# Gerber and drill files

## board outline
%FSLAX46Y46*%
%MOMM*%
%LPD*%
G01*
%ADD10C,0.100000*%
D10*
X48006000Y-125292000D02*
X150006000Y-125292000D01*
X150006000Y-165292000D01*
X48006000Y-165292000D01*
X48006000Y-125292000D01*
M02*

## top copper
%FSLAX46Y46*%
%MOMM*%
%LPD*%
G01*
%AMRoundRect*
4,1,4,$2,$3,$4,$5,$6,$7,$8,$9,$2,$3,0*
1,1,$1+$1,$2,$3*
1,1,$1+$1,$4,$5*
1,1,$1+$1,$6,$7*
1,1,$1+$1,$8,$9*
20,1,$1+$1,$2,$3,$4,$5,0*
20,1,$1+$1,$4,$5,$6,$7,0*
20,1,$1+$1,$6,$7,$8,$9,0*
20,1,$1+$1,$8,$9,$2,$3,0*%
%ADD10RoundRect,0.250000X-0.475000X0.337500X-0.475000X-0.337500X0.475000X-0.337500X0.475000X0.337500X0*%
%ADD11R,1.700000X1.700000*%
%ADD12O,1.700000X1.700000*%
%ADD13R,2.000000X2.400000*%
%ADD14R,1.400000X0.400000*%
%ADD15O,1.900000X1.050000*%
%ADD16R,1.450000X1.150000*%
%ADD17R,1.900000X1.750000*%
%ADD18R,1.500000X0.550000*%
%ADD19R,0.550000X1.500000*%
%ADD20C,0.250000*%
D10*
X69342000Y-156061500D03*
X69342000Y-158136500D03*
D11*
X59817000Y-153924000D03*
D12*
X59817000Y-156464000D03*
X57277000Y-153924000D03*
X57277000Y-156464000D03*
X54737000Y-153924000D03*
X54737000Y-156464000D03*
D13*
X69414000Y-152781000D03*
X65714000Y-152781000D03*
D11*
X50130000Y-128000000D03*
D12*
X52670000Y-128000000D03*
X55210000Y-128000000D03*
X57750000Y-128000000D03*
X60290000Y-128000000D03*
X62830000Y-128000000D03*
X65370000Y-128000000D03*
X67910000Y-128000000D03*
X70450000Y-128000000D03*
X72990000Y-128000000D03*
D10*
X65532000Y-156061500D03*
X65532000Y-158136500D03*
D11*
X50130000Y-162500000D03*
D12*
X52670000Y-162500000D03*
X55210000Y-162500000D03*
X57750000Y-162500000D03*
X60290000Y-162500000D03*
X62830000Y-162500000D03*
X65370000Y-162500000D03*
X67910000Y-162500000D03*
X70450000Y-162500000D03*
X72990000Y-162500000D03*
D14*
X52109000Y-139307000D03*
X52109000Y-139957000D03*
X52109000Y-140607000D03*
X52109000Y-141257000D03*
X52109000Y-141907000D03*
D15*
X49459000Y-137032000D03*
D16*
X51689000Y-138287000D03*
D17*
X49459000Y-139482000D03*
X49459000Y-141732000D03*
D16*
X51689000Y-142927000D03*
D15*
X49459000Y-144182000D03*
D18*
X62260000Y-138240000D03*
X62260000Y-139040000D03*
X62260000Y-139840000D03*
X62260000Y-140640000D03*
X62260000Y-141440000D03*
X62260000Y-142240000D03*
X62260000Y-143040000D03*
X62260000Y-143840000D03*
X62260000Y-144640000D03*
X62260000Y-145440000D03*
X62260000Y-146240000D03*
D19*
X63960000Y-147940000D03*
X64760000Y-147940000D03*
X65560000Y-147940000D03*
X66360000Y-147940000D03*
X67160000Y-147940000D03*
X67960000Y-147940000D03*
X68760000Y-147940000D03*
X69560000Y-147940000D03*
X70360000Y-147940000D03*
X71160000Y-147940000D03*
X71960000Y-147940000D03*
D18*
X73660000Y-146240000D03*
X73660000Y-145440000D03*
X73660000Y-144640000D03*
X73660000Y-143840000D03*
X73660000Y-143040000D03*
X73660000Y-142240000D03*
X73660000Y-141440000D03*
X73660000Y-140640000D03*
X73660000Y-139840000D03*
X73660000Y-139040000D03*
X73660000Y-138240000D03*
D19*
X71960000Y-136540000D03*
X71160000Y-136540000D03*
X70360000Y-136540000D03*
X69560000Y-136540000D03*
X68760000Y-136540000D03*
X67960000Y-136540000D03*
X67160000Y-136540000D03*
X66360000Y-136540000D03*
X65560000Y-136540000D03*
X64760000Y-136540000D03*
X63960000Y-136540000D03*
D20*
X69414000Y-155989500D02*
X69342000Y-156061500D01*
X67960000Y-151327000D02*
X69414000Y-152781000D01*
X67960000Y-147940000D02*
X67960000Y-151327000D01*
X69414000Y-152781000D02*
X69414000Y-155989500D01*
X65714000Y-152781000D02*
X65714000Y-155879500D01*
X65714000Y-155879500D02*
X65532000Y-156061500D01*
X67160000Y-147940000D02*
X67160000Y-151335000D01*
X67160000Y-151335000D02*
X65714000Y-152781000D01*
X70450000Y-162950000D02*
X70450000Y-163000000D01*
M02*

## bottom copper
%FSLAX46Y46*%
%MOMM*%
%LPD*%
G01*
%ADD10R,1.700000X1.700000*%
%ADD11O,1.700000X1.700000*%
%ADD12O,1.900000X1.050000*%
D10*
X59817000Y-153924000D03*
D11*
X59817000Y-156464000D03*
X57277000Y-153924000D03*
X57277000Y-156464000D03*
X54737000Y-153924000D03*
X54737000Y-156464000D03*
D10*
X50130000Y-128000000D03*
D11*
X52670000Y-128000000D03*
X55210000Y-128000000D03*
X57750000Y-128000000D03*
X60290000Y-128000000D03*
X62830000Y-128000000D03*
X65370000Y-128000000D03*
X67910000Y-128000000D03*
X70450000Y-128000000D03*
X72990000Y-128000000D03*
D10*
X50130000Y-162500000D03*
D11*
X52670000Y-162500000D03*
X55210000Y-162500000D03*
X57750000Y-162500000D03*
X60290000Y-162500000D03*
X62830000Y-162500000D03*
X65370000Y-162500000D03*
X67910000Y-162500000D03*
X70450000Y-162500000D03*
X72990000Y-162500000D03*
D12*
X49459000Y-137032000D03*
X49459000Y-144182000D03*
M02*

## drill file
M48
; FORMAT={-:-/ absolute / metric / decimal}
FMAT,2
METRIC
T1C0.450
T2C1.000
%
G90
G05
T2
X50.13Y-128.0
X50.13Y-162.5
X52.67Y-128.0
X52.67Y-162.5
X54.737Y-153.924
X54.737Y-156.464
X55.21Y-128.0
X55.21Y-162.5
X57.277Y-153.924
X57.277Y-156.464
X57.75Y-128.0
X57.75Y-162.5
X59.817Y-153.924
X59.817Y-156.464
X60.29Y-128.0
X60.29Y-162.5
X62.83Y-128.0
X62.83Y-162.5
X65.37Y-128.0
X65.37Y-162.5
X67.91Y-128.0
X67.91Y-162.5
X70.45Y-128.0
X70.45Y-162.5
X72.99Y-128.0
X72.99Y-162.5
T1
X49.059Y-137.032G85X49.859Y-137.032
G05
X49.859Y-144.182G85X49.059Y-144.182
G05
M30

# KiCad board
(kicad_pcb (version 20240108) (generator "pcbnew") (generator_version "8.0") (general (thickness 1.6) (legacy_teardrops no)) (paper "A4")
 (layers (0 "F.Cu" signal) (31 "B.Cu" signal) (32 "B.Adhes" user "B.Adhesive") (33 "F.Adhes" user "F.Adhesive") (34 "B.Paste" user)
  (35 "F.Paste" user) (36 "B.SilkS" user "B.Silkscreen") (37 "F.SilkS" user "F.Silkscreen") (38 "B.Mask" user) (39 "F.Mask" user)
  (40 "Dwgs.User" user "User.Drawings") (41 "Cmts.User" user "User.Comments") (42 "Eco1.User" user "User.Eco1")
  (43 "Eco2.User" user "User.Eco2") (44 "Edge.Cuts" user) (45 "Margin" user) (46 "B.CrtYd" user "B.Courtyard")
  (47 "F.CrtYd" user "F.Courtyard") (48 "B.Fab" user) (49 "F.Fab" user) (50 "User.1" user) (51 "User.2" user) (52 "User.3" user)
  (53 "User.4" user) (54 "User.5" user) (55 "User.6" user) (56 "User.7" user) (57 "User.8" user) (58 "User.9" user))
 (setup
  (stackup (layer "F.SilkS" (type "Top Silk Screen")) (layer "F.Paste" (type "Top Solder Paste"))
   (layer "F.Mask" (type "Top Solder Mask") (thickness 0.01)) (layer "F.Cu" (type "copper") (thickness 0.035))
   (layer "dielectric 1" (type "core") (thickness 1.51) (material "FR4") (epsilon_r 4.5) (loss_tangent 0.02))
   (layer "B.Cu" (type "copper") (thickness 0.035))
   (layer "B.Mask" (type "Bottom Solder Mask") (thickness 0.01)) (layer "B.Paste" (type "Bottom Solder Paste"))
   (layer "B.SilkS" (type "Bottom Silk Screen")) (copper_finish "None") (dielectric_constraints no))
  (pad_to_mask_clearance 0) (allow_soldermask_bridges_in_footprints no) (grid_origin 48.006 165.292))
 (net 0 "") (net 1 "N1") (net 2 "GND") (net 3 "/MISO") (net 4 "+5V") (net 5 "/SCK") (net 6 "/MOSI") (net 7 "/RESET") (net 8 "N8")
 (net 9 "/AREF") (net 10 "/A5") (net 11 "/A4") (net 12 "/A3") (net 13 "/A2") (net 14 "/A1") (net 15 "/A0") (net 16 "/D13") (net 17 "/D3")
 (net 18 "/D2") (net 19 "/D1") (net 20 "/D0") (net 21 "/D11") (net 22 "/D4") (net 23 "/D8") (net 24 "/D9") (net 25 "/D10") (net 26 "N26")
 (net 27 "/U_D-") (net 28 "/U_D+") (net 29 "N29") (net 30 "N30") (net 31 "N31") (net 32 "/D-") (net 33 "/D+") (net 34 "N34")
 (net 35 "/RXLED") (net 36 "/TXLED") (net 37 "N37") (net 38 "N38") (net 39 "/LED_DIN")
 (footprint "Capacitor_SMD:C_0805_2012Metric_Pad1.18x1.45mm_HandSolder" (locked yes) (layer "F.Cu") (at 69.342 157.099 -90)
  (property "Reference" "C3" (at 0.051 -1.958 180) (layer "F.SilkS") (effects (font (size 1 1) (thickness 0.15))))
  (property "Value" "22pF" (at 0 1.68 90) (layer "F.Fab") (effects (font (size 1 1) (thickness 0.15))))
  (pad "1" smd roundrect (at -1.0375 0 270) (size 1.175 1.45) (layers "F.Cu" "F.Paste" "F.Mask") (roundrect_rratio 0.2127659574)
   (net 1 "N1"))
  (pad "2" smd roundrect (at 1.0375 0 270) (size 1.175 1.45) (layers "F.Cu" "F.Paste" "F.Mask") (roundrect_rratio 0.2127659574)
   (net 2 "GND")))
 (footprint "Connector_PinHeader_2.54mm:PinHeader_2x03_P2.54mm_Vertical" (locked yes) (layer "F.Cu") (at 59.817 153.924 -90)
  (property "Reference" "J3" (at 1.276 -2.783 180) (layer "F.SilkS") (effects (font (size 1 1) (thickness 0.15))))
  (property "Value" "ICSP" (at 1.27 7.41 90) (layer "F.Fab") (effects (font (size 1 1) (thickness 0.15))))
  (pad "1" thru_hole rect (at 0 0 270) (size 1.7 1.7) (drill 1) (layers "*.Cu" "*.Mask") (remove_unused_layers no) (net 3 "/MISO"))
  (pad "2" thru_hole oval (at 2.54 0 270) (size 1.7 1.7) (drill 1) (layers "*.Cu" "*.Mask") (remove_unused_layers no) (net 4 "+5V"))
  (pad "3" thru_hole oval (at 0 2.54 270) (size 1.7 1.7) (drill 1) (layers "*.Cu" "*.Mask") (remove_unused_layers no) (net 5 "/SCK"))
  (pad "4" thru_hole oval (at 2.54 2.54 270) (size 1.7 1.7) (drill 1) (layers "*.Cu" "*.Mask") (remove_unused_layers no) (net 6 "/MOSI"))
  (pad "5" thru_hole oval (at 0 5.08 270) (size 1.7 1.7) (drill 1) (layers "*.Cu" "*.Mask") (remove_unused_layers no) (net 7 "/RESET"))
  (pad "6" thru_hole oval (at 2.54 5.08 270) (size 1.7 1.7) (drill 1) (layers "*.Cu" "*.Mask") (remove_unused_layers no) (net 2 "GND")))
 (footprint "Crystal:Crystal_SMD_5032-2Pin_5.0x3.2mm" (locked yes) (layer "F.Cu") (at 67.564 152.781 180)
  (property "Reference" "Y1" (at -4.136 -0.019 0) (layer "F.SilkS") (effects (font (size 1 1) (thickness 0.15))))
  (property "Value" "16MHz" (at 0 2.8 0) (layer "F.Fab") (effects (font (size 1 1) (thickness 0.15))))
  (pad "1" smd rect (at -1.85 0 180) (size 2 2.4) (layers "F.Cu" "F.Paste" "F.Mask") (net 1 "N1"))
  (pad "2" smd rect (at 1.85 0 180) (size 2 2.4) (layers "F.Cu" "F.Paste" "F.Mask") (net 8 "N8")))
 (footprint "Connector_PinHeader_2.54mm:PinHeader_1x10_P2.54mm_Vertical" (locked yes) (layer "F.Cu") (at 50.13 128 90)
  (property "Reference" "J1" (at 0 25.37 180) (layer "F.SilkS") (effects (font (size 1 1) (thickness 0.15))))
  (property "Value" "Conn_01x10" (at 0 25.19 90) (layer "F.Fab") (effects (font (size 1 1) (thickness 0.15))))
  (pad "1" thru_hole rect (at 0 0 90) (size 1.7 1.7) (drill 1) (layers "*.Cu" "*.Mask") (remove_unused_layers no) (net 4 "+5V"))
  (pad "2" thru_hole oval (at 0 2.54 90) (size 1.7 1.7) (drill 1) (layers "*.Cu" "*.Mask") (remove_unused_layers no) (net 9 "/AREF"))
  (pad "3" thru_hole oval (at 0 5.08 90) (size 1.7 1.7) (drill 1) (layers "*.Cu" "*.Mask") (remove_unused_layers no) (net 2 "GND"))
  (pad "4" thru_hole oval (at 0 7.62 90) (size 1.7 1.7) (drill 1) (layers "*.Cu" "*.Mask") (remove_unused_layers no) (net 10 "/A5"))
  (pad "5" thru_hole oval (at 0 10.16 90) (size 1.7 1.7) (drill 1) (layers "*.Cu" "*.Mask") (remove_unused_layers no) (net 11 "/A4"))
  (pad "6" thru_hole oval (at 0 12.7 90) (size 1.7 1.7) (drill 1) (layers "*.Cu" "*.Mask") (remove_unused_layers no) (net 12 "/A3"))
  (pad "7" thru_hole oval (at 0 15.24 90) (size 1.7 1.7) (drill 1) (layers "*.Cu" "*.Mask") (remove_unused_layers no) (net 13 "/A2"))
  (pad "8" thru_hole oval (at 0 17.78 90) (size 1.7 1.7) (drill 1) (layers "*.Cu" "*.Mask") (remove_unused_layers no) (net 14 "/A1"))
  (pad "9" thru_hole oval (at 0 20.32 90) (size 1.7 1.7) (drill 1) (layers "*.Cu" "*.Mask") (remove_unused_layers no) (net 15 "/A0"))
  (pad "10" thru_hole oval (at 0 22.86 90) (size 1.7 1.7) (drill 1) (layers "*.Cu" "*.Mask") (remove_unused_layers no) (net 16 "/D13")))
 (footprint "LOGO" (layer "F.Cu") (at 142.15 161.8)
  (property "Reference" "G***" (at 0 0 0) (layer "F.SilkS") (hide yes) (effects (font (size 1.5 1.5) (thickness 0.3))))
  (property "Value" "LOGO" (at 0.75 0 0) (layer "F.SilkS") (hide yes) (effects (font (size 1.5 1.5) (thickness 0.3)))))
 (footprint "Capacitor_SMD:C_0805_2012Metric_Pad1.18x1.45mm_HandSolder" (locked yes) (layer "F.Cu") (at 65.532 157.099 -90)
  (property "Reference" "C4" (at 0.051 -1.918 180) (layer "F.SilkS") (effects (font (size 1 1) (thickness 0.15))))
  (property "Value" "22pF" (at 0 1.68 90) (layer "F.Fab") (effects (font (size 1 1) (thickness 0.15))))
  (pad "1" smd roundrect (at -1.0375 0 270) (size 1.175 1.45) (layers "F.Cu" "F.Paste" "F.Mask") (roundrect_rratio 0.2127659574)
   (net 8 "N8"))
  (pad "2" smd roundrect (at 1.0375 0 270) (size 1.175 1.45) (layers "F.Cu" "F.Paste" "F.Mask") (roundrect_rratio 0.2127659574)
   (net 2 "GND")))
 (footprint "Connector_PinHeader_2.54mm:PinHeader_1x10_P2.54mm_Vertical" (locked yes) (layer "F.Cu") (at 50.13 162.5 90)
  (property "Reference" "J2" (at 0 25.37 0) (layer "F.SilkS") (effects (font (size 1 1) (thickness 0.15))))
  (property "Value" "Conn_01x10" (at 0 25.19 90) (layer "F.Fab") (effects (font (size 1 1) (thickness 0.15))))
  (pad "1" thru_hole rect (at 0 0 90) (size 1.7 1.7) (drill 1) (layers "*.Cu" "*.Mask") (remove_unused_layers no) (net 2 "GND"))
  (pad "2" thru_hole oval (at 0 2.54 90) (size 1.7 1.7) (drill 1) (layers "*.Cu" "*.Mask") (remove_unused_layers no) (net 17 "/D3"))
  (pad "3" thru_hole oval (at 0 5.08 90) (size 1.7 1.7) (drill 1) (layers "*.Cu" "*.Mask") (remove_unused_layers no) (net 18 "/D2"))
  (pad "4" thru_hole oval (at 0 7.62 90) (size 1.7 1.7) (drill 1) (layers "*.Cu" "*.Mask") (remove_unused_layers no) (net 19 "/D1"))
  (pad "5" thru_hole oval (at 0 10.16 90) (size 1.7 1.7) (drill 1) (layers "*.Cu" "*.Mask") (remove_unused_layers no) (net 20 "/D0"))
  (pad "6" thru_hole oval (at 0 12.7 90) (size 1.7 1.7) (drill 1) (layers "*.Cu" "*.Mask") (remove_unused_layers no) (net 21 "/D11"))
  (pad "7" thru_hole oval (at 0 15.24 90) (size 1.7 1.7) (drill 1) (layers "*.Cu" "*.Mask") (remove_unused_layers no) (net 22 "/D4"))
  (pad "8" thru_hole oval (at 0 17.78 90) (size 1.7 1.7) (drill 1) (layers "*.Cu" "*.Mask") (remove_unused_layers no) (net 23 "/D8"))
  (pad "9" thru_hole oval (at 0 20.32 90) (size 1.7 1.7) (drill 1) (layers "*.Cu" "*.Mask") (remove_unused_layers no) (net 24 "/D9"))
  (pad "10" thru_hole oval (at 0 22.86 90) (size 1.7 1.7) (drill 1) (layers "*.Cu" "*.Mask") (remove_unused_layers no) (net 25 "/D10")))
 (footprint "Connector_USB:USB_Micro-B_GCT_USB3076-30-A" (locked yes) (layer "F.Cu") (at 50.659 140.607 -90)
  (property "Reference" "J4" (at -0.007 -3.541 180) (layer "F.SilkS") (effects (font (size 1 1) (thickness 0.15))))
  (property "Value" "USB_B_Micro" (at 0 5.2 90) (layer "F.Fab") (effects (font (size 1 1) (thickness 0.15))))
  (pad "1" smd rect (at -1.3 -1.45 270) (size 0.4 1.4) (layers "F.Cu" "F.Paste" "F.Mask") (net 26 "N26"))
  (pad "2" smd rect (at -0.65 -1.45 270) (size 0.4 1.4) (layers "F.Cu" "F.Paste" "F.Mask") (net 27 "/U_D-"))
  (pad "3" smd rect (at 0 -1.45 270) (size 0.4 1.4) (layers "F.Cu" "F.Paste" "F.Mask") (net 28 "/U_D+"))
  (pad "4" smd rect (at 0.65 -1.45 270) (size 0.4 1.4) (layers "F.Cu" "F.Paste" "F.Mask") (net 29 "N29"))
  (pad "5" smd rect (at 1.3 -1.45 270) (size 0.4 1.4) (layers "F.Cu" "F.Paste" "F.Mask") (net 2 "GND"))
  (pad "6" thru_hole oval (at -3.575 1.2 90) (size 1.05 1.9) (drill oval 0.45 1.25) (layers "*.Cu" "*.Mask") (remove_unused_layers no)
   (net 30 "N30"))
  (pad "6" smd rect (at -2.32 -1.03 270) (size 1.15 1.45) (layers "F.Cu" "F.Paste" "F.Mask") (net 30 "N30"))
  (pad "6" smd rect (at -1.125 1.2 270) (size 1.75 1.9) (layers "F.Cu" "F.Paste" "F.Mask") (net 30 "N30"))
  (pad "6" smd rect (at 1.125 1.2 270) (size 1.75 1.9) (layers "F.Cu" "F.Paste" "F.Mask") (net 30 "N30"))
  (pad "6" smd rect (at 2.32 -1.03 270) (size 1.15 1.45) (layers "F.Cu" "F.Paste" "F.Mask") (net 30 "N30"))
  (pad "6" thru_hole oval (at 3.575 1.2 270) (size 1.05 1.9) (drill oval 0.45 1.25) (layers "*.Cu" "*.Mask") (remove_unused_layers no)
   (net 30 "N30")))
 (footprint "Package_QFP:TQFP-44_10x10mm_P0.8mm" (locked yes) (layer "F.Cu") (at 67.96 142.24)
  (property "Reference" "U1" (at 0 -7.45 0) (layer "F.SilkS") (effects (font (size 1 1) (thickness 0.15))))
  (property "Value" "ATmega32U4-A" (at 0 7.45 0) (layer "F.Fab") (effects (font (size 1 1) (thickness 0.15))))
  (pad "1" smd rect (at -5.7 -4) (size 1.5 0.55) (layers "F.Cu" "F.Paste" "F.Mask") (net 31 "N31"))
  (pad "2" smd rect (at -5.7 -3.2) (size 1.5 0.55) (layers "F.Cu" "F.Paste" "F.Mask") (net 4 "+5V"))
  (pad "3" smd rect (at -5.7 -2.4) (size 1.5 0.55) (layers "F.Cu" "F.Paste" "F.Mask") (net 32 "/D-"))
  (pad "4" smd rect (at -5.7 -1.6) (size 1.5 0.55) (layers "F.Cu" "F.Paste" "F.Mask") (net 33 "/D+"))
  (pad "5" smd rect (at -5.7 -0.8) (size 1.5 0.55) (layers "F.Cu" "F.Paste" "F.Mask") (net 2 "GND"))
  (pad "6" smd rect (at -5.7 0) (size 1.5 0.55) (layers "F.Cu" "F.Paste" "F.Mask") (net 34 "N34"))
  (pad "7" smd rect (at -5.7 0.8) (size 1.5 0.55) (layers "F.Cu" "F.Paste" "F.Mask") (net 4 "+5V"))
  (pad "8" smd rect (at -5.7 1.6) (size 1.5 0.55) (layers "F.Cu" "F.Paste" "F.Mask") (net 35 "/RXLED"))
  (pad "9" smd rect (at -5.7 2.4) (size 1.5 0.55) (layers "F.Cu" "F.Paste" "F.Mask") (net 5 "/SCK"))
  (pad "10" smd rect (at -5.7 3.2) (size 1.5 0.55) (layers "F.Cu" "F.Paste" "F.Mask") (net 6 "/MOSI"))
  (pad "11" smd rect (at -5.7 4) (size 1.5 0.55) (layers "F.Cu" "F.Paste" "F.Mask") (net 3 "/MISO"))
  (pad "12" smd rect (at -4 5.7 90) (size 1.5 0.55) (layers "F.Cu" "F.Paste" "F.Mask") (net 21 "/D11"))
  (pad "13" smd rect (at -3.2 5.7 90) (size 1.5 0.55) (layers "F.Cu" "F.Paste" "F.Mask") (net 7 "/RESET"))
  (pad "14" smd rect (at -2.4 5.7 90) (size 1.5 0.55) (layers "F.Cu" "F.Paste" "F.Mask") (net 4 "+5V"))
  (pad "15" smd rect (at -1.6 5.7 90) (size 1.5 0.55) (layers "F.Cu" "F.Paste" "F.Mask") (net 2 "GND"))
  (pad "16" smd rect (at -0.8 5.7 90) (size 1.5 0.55) (layers "F.Cu" "F.Paste" "F.Mask") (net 8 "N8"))
  (pad "17" smd rect (at 0 5.7 90) (size 1.5 0.55) (layers "F.Cu" "F.Paste" "F.Mask") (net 1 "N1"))
  (pad "18" smd rect (at 0.8 5.7 90) (size 1.5 0.55) (layers "F.Cu" "F.Paste" "F.Mask") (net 17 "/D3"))
  (pad "19" smd rect (at 1.6 5.7 90) (size 1.5 0.55) (layers "F.Cu" "F.Paste" "F.Mask") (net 18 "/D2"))
  (pad "20" smd rect (at 2.4 5.7 90) (size 1.5 0.55) (layers "F.Cu" "F.Paste" "F.Mask") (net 20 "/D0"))
  (pad "21" smd rect (at 3.2 5.7 90) (size 1.5 0.55) (layers "F.Cu" "F.Paste" "F.Mask") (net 19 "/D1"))
  (pad "22" smd rect (at 4 5.7 90) (size 1.5 0.55) (layers "F.Cu" "F.Paste" "F.Mask") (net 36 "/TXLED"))
  (pad "23" smd rect (at 5.7 4) (size 1.5 0.55) (layers "F.Cu" "F.Paste" "F.Mask") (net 2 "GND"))
  (pad "24" smd rect (at 5.7 3.2) (size 1.5 0.55) (layers "F.Cu" "F.Paste" "F.Mask") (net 4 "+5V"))
  (pad "25" smd rect (at 5.7 2.4) (size 1.5 0.55) (layers "F.Cu" "F.Paste" "F.Mask") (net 22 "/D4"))
  (pad "26" smd rect (at 5.7 1.6) (size 1.5 0.55) (layers "F.Cu" "F.Paste" "F.Mask") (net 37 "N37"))
  (pad "27" smd rect (at 5.7 0.8) (size 1.5 0.55) (layers "F.Cu" "F.Paste" "F.Mask") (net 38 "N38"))
  (pad "28" smd rect (at 5.7 0) (size 1.5 0.55) (layers "F.Cu" "F.Paste" "F.Mask") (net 23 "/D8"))
  (pad "29" smd rect (at 5.7 -0.8) (size 1.5 0.55) (layers "F.Cu" "F.Paste" "F.Mask") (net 24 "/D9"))
  (pad "30" smd rect (at 5.7 -1.6) (size 1.5 0.55) (layers "F.Cu" "F.Paste" "F.Mask") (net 25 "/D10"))
  (pad "31" smd rect (at 5.7 -2.4) (size 1.5 0.55) (layers "F.Cu" "F.Paste" "F.Mask") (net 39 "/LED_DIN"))
  (pad "32" smd rect (at 5.7 -3.2) (size 1.5 0.55) (layers "F.Cu" "F.Paste" "F.Mask") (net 16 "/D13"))
  (pad "33" smd rect (at 5.7 -4) (size 1.5 0.55) (layers "F.Cu" "F.Paste" "F.Mask") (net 2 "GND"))
  (pad "34" smd rect (at 4 -5.7 90) (size 1.5 0.55) (layers "F.Cu" "F.Paste" "F.Mask") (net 4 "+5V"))
  (pad "35" smd rect (at 3.2 -5.7 90) (size 1.5 0.55) (layers "F.Cu" "F.Paste" "F.Mask") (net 2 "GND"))
  (pad "36" smd rect (at 2.4 -5.7 90) (size 1.5 0.55) (layers "F.Cu" "F.Paste" "F.Mask") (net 15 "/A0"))
  (pad "37" smd rect (at 1.6 -5.7 90) (size 1.5 0.55) (layers "F.Cu" "F.Paste" "F.Mask") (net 14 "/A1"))
  (pad "38" smd rect (at 0.8 -5.7 90) (size 1.5 0.55) (layers "F.Cu" "F.Paste" "F.Mask") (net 13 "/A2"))
  (pad "39" smd rect (at 0 -5.7 90) (size 1.5 0.55) (layers "F.Cu" "F.Paste" "F.Mask") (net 12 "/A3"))
  (pad "40" smd rect (at -0.8 -5.7 90) (size 1.5 0.55) (layers "F.Cu" "F.Paste" "F.Mask") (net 11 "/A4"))
  (pad "41" smd rect (at -1.6 -5.7 90) (size 1.5 0.55) (layers "F.Cu" "F.Paste" "F.Mask") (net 10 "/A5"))
  (pad "42" smd rect (at -2.4 -5.7 90) (size 1.5 0.55) (layers "F.Cu" "F.Paste" "F.Mask") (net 9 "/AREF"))
  (pad "43" smd rect (at -3.2 -5.7 90) (size 1.5 0.55) (layers "F.Cu" "F.Paste" "F.Mask") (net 2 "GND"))
  (pad "44" smd rect (at -4 -5.7 90) (size 1.5 0.55) (layers "F.Cu" "F.Paste" "F.Mask") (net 4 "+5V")))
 (gr_rect (start 48.006 125.292) (end 150.006 165.292) (locked yes) (stroke (width 0.1) (type default)) (fill none) (layer "Edge.Cuts"))
 (segment (start 69.414 155.9895) (end 69.342 156.0615) (width 0.25) (locked yes) (layer "F.Cu") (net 1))
 (segment (start 67.96 151.327) (end 69.414 152.781) (width 0.25) (locked yes) (layer "F.Cu") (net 1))
 (segment (start 67.96 147.94) (end 67.96 151.327) (width 0.25) (locked yes) (layer "F.Cu") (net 1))
 (segment (start 69.414 152.781) (end 69.414 155.9895) (width 0.25) (locked yes) (layer "F.Cu") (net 1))
 (segment (start 65.714 152.781) (end 65.714 155.8795) (width 0.25) (locked yes) (layer "F.Cu") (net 8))
 (segment (start 65.714 155.8795) (end 65.532 156.0615) (width 0.25) (locked yes) (layer "F.Cu") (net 8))
 (segment (start 67.16 147.94) (end 67.16 151.335) (width 0.25) (locked yes) (layer "F.Cu") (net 8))
 (segment (start 67.16 151.335) (end 65.714 152.781) (width 0.25) (locked yes) (layer "F.Cu") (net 8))
 (segment (start 70.45 162.95) (end 70.45 163) (width 0.25) (layer "F.Cu") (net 24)))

